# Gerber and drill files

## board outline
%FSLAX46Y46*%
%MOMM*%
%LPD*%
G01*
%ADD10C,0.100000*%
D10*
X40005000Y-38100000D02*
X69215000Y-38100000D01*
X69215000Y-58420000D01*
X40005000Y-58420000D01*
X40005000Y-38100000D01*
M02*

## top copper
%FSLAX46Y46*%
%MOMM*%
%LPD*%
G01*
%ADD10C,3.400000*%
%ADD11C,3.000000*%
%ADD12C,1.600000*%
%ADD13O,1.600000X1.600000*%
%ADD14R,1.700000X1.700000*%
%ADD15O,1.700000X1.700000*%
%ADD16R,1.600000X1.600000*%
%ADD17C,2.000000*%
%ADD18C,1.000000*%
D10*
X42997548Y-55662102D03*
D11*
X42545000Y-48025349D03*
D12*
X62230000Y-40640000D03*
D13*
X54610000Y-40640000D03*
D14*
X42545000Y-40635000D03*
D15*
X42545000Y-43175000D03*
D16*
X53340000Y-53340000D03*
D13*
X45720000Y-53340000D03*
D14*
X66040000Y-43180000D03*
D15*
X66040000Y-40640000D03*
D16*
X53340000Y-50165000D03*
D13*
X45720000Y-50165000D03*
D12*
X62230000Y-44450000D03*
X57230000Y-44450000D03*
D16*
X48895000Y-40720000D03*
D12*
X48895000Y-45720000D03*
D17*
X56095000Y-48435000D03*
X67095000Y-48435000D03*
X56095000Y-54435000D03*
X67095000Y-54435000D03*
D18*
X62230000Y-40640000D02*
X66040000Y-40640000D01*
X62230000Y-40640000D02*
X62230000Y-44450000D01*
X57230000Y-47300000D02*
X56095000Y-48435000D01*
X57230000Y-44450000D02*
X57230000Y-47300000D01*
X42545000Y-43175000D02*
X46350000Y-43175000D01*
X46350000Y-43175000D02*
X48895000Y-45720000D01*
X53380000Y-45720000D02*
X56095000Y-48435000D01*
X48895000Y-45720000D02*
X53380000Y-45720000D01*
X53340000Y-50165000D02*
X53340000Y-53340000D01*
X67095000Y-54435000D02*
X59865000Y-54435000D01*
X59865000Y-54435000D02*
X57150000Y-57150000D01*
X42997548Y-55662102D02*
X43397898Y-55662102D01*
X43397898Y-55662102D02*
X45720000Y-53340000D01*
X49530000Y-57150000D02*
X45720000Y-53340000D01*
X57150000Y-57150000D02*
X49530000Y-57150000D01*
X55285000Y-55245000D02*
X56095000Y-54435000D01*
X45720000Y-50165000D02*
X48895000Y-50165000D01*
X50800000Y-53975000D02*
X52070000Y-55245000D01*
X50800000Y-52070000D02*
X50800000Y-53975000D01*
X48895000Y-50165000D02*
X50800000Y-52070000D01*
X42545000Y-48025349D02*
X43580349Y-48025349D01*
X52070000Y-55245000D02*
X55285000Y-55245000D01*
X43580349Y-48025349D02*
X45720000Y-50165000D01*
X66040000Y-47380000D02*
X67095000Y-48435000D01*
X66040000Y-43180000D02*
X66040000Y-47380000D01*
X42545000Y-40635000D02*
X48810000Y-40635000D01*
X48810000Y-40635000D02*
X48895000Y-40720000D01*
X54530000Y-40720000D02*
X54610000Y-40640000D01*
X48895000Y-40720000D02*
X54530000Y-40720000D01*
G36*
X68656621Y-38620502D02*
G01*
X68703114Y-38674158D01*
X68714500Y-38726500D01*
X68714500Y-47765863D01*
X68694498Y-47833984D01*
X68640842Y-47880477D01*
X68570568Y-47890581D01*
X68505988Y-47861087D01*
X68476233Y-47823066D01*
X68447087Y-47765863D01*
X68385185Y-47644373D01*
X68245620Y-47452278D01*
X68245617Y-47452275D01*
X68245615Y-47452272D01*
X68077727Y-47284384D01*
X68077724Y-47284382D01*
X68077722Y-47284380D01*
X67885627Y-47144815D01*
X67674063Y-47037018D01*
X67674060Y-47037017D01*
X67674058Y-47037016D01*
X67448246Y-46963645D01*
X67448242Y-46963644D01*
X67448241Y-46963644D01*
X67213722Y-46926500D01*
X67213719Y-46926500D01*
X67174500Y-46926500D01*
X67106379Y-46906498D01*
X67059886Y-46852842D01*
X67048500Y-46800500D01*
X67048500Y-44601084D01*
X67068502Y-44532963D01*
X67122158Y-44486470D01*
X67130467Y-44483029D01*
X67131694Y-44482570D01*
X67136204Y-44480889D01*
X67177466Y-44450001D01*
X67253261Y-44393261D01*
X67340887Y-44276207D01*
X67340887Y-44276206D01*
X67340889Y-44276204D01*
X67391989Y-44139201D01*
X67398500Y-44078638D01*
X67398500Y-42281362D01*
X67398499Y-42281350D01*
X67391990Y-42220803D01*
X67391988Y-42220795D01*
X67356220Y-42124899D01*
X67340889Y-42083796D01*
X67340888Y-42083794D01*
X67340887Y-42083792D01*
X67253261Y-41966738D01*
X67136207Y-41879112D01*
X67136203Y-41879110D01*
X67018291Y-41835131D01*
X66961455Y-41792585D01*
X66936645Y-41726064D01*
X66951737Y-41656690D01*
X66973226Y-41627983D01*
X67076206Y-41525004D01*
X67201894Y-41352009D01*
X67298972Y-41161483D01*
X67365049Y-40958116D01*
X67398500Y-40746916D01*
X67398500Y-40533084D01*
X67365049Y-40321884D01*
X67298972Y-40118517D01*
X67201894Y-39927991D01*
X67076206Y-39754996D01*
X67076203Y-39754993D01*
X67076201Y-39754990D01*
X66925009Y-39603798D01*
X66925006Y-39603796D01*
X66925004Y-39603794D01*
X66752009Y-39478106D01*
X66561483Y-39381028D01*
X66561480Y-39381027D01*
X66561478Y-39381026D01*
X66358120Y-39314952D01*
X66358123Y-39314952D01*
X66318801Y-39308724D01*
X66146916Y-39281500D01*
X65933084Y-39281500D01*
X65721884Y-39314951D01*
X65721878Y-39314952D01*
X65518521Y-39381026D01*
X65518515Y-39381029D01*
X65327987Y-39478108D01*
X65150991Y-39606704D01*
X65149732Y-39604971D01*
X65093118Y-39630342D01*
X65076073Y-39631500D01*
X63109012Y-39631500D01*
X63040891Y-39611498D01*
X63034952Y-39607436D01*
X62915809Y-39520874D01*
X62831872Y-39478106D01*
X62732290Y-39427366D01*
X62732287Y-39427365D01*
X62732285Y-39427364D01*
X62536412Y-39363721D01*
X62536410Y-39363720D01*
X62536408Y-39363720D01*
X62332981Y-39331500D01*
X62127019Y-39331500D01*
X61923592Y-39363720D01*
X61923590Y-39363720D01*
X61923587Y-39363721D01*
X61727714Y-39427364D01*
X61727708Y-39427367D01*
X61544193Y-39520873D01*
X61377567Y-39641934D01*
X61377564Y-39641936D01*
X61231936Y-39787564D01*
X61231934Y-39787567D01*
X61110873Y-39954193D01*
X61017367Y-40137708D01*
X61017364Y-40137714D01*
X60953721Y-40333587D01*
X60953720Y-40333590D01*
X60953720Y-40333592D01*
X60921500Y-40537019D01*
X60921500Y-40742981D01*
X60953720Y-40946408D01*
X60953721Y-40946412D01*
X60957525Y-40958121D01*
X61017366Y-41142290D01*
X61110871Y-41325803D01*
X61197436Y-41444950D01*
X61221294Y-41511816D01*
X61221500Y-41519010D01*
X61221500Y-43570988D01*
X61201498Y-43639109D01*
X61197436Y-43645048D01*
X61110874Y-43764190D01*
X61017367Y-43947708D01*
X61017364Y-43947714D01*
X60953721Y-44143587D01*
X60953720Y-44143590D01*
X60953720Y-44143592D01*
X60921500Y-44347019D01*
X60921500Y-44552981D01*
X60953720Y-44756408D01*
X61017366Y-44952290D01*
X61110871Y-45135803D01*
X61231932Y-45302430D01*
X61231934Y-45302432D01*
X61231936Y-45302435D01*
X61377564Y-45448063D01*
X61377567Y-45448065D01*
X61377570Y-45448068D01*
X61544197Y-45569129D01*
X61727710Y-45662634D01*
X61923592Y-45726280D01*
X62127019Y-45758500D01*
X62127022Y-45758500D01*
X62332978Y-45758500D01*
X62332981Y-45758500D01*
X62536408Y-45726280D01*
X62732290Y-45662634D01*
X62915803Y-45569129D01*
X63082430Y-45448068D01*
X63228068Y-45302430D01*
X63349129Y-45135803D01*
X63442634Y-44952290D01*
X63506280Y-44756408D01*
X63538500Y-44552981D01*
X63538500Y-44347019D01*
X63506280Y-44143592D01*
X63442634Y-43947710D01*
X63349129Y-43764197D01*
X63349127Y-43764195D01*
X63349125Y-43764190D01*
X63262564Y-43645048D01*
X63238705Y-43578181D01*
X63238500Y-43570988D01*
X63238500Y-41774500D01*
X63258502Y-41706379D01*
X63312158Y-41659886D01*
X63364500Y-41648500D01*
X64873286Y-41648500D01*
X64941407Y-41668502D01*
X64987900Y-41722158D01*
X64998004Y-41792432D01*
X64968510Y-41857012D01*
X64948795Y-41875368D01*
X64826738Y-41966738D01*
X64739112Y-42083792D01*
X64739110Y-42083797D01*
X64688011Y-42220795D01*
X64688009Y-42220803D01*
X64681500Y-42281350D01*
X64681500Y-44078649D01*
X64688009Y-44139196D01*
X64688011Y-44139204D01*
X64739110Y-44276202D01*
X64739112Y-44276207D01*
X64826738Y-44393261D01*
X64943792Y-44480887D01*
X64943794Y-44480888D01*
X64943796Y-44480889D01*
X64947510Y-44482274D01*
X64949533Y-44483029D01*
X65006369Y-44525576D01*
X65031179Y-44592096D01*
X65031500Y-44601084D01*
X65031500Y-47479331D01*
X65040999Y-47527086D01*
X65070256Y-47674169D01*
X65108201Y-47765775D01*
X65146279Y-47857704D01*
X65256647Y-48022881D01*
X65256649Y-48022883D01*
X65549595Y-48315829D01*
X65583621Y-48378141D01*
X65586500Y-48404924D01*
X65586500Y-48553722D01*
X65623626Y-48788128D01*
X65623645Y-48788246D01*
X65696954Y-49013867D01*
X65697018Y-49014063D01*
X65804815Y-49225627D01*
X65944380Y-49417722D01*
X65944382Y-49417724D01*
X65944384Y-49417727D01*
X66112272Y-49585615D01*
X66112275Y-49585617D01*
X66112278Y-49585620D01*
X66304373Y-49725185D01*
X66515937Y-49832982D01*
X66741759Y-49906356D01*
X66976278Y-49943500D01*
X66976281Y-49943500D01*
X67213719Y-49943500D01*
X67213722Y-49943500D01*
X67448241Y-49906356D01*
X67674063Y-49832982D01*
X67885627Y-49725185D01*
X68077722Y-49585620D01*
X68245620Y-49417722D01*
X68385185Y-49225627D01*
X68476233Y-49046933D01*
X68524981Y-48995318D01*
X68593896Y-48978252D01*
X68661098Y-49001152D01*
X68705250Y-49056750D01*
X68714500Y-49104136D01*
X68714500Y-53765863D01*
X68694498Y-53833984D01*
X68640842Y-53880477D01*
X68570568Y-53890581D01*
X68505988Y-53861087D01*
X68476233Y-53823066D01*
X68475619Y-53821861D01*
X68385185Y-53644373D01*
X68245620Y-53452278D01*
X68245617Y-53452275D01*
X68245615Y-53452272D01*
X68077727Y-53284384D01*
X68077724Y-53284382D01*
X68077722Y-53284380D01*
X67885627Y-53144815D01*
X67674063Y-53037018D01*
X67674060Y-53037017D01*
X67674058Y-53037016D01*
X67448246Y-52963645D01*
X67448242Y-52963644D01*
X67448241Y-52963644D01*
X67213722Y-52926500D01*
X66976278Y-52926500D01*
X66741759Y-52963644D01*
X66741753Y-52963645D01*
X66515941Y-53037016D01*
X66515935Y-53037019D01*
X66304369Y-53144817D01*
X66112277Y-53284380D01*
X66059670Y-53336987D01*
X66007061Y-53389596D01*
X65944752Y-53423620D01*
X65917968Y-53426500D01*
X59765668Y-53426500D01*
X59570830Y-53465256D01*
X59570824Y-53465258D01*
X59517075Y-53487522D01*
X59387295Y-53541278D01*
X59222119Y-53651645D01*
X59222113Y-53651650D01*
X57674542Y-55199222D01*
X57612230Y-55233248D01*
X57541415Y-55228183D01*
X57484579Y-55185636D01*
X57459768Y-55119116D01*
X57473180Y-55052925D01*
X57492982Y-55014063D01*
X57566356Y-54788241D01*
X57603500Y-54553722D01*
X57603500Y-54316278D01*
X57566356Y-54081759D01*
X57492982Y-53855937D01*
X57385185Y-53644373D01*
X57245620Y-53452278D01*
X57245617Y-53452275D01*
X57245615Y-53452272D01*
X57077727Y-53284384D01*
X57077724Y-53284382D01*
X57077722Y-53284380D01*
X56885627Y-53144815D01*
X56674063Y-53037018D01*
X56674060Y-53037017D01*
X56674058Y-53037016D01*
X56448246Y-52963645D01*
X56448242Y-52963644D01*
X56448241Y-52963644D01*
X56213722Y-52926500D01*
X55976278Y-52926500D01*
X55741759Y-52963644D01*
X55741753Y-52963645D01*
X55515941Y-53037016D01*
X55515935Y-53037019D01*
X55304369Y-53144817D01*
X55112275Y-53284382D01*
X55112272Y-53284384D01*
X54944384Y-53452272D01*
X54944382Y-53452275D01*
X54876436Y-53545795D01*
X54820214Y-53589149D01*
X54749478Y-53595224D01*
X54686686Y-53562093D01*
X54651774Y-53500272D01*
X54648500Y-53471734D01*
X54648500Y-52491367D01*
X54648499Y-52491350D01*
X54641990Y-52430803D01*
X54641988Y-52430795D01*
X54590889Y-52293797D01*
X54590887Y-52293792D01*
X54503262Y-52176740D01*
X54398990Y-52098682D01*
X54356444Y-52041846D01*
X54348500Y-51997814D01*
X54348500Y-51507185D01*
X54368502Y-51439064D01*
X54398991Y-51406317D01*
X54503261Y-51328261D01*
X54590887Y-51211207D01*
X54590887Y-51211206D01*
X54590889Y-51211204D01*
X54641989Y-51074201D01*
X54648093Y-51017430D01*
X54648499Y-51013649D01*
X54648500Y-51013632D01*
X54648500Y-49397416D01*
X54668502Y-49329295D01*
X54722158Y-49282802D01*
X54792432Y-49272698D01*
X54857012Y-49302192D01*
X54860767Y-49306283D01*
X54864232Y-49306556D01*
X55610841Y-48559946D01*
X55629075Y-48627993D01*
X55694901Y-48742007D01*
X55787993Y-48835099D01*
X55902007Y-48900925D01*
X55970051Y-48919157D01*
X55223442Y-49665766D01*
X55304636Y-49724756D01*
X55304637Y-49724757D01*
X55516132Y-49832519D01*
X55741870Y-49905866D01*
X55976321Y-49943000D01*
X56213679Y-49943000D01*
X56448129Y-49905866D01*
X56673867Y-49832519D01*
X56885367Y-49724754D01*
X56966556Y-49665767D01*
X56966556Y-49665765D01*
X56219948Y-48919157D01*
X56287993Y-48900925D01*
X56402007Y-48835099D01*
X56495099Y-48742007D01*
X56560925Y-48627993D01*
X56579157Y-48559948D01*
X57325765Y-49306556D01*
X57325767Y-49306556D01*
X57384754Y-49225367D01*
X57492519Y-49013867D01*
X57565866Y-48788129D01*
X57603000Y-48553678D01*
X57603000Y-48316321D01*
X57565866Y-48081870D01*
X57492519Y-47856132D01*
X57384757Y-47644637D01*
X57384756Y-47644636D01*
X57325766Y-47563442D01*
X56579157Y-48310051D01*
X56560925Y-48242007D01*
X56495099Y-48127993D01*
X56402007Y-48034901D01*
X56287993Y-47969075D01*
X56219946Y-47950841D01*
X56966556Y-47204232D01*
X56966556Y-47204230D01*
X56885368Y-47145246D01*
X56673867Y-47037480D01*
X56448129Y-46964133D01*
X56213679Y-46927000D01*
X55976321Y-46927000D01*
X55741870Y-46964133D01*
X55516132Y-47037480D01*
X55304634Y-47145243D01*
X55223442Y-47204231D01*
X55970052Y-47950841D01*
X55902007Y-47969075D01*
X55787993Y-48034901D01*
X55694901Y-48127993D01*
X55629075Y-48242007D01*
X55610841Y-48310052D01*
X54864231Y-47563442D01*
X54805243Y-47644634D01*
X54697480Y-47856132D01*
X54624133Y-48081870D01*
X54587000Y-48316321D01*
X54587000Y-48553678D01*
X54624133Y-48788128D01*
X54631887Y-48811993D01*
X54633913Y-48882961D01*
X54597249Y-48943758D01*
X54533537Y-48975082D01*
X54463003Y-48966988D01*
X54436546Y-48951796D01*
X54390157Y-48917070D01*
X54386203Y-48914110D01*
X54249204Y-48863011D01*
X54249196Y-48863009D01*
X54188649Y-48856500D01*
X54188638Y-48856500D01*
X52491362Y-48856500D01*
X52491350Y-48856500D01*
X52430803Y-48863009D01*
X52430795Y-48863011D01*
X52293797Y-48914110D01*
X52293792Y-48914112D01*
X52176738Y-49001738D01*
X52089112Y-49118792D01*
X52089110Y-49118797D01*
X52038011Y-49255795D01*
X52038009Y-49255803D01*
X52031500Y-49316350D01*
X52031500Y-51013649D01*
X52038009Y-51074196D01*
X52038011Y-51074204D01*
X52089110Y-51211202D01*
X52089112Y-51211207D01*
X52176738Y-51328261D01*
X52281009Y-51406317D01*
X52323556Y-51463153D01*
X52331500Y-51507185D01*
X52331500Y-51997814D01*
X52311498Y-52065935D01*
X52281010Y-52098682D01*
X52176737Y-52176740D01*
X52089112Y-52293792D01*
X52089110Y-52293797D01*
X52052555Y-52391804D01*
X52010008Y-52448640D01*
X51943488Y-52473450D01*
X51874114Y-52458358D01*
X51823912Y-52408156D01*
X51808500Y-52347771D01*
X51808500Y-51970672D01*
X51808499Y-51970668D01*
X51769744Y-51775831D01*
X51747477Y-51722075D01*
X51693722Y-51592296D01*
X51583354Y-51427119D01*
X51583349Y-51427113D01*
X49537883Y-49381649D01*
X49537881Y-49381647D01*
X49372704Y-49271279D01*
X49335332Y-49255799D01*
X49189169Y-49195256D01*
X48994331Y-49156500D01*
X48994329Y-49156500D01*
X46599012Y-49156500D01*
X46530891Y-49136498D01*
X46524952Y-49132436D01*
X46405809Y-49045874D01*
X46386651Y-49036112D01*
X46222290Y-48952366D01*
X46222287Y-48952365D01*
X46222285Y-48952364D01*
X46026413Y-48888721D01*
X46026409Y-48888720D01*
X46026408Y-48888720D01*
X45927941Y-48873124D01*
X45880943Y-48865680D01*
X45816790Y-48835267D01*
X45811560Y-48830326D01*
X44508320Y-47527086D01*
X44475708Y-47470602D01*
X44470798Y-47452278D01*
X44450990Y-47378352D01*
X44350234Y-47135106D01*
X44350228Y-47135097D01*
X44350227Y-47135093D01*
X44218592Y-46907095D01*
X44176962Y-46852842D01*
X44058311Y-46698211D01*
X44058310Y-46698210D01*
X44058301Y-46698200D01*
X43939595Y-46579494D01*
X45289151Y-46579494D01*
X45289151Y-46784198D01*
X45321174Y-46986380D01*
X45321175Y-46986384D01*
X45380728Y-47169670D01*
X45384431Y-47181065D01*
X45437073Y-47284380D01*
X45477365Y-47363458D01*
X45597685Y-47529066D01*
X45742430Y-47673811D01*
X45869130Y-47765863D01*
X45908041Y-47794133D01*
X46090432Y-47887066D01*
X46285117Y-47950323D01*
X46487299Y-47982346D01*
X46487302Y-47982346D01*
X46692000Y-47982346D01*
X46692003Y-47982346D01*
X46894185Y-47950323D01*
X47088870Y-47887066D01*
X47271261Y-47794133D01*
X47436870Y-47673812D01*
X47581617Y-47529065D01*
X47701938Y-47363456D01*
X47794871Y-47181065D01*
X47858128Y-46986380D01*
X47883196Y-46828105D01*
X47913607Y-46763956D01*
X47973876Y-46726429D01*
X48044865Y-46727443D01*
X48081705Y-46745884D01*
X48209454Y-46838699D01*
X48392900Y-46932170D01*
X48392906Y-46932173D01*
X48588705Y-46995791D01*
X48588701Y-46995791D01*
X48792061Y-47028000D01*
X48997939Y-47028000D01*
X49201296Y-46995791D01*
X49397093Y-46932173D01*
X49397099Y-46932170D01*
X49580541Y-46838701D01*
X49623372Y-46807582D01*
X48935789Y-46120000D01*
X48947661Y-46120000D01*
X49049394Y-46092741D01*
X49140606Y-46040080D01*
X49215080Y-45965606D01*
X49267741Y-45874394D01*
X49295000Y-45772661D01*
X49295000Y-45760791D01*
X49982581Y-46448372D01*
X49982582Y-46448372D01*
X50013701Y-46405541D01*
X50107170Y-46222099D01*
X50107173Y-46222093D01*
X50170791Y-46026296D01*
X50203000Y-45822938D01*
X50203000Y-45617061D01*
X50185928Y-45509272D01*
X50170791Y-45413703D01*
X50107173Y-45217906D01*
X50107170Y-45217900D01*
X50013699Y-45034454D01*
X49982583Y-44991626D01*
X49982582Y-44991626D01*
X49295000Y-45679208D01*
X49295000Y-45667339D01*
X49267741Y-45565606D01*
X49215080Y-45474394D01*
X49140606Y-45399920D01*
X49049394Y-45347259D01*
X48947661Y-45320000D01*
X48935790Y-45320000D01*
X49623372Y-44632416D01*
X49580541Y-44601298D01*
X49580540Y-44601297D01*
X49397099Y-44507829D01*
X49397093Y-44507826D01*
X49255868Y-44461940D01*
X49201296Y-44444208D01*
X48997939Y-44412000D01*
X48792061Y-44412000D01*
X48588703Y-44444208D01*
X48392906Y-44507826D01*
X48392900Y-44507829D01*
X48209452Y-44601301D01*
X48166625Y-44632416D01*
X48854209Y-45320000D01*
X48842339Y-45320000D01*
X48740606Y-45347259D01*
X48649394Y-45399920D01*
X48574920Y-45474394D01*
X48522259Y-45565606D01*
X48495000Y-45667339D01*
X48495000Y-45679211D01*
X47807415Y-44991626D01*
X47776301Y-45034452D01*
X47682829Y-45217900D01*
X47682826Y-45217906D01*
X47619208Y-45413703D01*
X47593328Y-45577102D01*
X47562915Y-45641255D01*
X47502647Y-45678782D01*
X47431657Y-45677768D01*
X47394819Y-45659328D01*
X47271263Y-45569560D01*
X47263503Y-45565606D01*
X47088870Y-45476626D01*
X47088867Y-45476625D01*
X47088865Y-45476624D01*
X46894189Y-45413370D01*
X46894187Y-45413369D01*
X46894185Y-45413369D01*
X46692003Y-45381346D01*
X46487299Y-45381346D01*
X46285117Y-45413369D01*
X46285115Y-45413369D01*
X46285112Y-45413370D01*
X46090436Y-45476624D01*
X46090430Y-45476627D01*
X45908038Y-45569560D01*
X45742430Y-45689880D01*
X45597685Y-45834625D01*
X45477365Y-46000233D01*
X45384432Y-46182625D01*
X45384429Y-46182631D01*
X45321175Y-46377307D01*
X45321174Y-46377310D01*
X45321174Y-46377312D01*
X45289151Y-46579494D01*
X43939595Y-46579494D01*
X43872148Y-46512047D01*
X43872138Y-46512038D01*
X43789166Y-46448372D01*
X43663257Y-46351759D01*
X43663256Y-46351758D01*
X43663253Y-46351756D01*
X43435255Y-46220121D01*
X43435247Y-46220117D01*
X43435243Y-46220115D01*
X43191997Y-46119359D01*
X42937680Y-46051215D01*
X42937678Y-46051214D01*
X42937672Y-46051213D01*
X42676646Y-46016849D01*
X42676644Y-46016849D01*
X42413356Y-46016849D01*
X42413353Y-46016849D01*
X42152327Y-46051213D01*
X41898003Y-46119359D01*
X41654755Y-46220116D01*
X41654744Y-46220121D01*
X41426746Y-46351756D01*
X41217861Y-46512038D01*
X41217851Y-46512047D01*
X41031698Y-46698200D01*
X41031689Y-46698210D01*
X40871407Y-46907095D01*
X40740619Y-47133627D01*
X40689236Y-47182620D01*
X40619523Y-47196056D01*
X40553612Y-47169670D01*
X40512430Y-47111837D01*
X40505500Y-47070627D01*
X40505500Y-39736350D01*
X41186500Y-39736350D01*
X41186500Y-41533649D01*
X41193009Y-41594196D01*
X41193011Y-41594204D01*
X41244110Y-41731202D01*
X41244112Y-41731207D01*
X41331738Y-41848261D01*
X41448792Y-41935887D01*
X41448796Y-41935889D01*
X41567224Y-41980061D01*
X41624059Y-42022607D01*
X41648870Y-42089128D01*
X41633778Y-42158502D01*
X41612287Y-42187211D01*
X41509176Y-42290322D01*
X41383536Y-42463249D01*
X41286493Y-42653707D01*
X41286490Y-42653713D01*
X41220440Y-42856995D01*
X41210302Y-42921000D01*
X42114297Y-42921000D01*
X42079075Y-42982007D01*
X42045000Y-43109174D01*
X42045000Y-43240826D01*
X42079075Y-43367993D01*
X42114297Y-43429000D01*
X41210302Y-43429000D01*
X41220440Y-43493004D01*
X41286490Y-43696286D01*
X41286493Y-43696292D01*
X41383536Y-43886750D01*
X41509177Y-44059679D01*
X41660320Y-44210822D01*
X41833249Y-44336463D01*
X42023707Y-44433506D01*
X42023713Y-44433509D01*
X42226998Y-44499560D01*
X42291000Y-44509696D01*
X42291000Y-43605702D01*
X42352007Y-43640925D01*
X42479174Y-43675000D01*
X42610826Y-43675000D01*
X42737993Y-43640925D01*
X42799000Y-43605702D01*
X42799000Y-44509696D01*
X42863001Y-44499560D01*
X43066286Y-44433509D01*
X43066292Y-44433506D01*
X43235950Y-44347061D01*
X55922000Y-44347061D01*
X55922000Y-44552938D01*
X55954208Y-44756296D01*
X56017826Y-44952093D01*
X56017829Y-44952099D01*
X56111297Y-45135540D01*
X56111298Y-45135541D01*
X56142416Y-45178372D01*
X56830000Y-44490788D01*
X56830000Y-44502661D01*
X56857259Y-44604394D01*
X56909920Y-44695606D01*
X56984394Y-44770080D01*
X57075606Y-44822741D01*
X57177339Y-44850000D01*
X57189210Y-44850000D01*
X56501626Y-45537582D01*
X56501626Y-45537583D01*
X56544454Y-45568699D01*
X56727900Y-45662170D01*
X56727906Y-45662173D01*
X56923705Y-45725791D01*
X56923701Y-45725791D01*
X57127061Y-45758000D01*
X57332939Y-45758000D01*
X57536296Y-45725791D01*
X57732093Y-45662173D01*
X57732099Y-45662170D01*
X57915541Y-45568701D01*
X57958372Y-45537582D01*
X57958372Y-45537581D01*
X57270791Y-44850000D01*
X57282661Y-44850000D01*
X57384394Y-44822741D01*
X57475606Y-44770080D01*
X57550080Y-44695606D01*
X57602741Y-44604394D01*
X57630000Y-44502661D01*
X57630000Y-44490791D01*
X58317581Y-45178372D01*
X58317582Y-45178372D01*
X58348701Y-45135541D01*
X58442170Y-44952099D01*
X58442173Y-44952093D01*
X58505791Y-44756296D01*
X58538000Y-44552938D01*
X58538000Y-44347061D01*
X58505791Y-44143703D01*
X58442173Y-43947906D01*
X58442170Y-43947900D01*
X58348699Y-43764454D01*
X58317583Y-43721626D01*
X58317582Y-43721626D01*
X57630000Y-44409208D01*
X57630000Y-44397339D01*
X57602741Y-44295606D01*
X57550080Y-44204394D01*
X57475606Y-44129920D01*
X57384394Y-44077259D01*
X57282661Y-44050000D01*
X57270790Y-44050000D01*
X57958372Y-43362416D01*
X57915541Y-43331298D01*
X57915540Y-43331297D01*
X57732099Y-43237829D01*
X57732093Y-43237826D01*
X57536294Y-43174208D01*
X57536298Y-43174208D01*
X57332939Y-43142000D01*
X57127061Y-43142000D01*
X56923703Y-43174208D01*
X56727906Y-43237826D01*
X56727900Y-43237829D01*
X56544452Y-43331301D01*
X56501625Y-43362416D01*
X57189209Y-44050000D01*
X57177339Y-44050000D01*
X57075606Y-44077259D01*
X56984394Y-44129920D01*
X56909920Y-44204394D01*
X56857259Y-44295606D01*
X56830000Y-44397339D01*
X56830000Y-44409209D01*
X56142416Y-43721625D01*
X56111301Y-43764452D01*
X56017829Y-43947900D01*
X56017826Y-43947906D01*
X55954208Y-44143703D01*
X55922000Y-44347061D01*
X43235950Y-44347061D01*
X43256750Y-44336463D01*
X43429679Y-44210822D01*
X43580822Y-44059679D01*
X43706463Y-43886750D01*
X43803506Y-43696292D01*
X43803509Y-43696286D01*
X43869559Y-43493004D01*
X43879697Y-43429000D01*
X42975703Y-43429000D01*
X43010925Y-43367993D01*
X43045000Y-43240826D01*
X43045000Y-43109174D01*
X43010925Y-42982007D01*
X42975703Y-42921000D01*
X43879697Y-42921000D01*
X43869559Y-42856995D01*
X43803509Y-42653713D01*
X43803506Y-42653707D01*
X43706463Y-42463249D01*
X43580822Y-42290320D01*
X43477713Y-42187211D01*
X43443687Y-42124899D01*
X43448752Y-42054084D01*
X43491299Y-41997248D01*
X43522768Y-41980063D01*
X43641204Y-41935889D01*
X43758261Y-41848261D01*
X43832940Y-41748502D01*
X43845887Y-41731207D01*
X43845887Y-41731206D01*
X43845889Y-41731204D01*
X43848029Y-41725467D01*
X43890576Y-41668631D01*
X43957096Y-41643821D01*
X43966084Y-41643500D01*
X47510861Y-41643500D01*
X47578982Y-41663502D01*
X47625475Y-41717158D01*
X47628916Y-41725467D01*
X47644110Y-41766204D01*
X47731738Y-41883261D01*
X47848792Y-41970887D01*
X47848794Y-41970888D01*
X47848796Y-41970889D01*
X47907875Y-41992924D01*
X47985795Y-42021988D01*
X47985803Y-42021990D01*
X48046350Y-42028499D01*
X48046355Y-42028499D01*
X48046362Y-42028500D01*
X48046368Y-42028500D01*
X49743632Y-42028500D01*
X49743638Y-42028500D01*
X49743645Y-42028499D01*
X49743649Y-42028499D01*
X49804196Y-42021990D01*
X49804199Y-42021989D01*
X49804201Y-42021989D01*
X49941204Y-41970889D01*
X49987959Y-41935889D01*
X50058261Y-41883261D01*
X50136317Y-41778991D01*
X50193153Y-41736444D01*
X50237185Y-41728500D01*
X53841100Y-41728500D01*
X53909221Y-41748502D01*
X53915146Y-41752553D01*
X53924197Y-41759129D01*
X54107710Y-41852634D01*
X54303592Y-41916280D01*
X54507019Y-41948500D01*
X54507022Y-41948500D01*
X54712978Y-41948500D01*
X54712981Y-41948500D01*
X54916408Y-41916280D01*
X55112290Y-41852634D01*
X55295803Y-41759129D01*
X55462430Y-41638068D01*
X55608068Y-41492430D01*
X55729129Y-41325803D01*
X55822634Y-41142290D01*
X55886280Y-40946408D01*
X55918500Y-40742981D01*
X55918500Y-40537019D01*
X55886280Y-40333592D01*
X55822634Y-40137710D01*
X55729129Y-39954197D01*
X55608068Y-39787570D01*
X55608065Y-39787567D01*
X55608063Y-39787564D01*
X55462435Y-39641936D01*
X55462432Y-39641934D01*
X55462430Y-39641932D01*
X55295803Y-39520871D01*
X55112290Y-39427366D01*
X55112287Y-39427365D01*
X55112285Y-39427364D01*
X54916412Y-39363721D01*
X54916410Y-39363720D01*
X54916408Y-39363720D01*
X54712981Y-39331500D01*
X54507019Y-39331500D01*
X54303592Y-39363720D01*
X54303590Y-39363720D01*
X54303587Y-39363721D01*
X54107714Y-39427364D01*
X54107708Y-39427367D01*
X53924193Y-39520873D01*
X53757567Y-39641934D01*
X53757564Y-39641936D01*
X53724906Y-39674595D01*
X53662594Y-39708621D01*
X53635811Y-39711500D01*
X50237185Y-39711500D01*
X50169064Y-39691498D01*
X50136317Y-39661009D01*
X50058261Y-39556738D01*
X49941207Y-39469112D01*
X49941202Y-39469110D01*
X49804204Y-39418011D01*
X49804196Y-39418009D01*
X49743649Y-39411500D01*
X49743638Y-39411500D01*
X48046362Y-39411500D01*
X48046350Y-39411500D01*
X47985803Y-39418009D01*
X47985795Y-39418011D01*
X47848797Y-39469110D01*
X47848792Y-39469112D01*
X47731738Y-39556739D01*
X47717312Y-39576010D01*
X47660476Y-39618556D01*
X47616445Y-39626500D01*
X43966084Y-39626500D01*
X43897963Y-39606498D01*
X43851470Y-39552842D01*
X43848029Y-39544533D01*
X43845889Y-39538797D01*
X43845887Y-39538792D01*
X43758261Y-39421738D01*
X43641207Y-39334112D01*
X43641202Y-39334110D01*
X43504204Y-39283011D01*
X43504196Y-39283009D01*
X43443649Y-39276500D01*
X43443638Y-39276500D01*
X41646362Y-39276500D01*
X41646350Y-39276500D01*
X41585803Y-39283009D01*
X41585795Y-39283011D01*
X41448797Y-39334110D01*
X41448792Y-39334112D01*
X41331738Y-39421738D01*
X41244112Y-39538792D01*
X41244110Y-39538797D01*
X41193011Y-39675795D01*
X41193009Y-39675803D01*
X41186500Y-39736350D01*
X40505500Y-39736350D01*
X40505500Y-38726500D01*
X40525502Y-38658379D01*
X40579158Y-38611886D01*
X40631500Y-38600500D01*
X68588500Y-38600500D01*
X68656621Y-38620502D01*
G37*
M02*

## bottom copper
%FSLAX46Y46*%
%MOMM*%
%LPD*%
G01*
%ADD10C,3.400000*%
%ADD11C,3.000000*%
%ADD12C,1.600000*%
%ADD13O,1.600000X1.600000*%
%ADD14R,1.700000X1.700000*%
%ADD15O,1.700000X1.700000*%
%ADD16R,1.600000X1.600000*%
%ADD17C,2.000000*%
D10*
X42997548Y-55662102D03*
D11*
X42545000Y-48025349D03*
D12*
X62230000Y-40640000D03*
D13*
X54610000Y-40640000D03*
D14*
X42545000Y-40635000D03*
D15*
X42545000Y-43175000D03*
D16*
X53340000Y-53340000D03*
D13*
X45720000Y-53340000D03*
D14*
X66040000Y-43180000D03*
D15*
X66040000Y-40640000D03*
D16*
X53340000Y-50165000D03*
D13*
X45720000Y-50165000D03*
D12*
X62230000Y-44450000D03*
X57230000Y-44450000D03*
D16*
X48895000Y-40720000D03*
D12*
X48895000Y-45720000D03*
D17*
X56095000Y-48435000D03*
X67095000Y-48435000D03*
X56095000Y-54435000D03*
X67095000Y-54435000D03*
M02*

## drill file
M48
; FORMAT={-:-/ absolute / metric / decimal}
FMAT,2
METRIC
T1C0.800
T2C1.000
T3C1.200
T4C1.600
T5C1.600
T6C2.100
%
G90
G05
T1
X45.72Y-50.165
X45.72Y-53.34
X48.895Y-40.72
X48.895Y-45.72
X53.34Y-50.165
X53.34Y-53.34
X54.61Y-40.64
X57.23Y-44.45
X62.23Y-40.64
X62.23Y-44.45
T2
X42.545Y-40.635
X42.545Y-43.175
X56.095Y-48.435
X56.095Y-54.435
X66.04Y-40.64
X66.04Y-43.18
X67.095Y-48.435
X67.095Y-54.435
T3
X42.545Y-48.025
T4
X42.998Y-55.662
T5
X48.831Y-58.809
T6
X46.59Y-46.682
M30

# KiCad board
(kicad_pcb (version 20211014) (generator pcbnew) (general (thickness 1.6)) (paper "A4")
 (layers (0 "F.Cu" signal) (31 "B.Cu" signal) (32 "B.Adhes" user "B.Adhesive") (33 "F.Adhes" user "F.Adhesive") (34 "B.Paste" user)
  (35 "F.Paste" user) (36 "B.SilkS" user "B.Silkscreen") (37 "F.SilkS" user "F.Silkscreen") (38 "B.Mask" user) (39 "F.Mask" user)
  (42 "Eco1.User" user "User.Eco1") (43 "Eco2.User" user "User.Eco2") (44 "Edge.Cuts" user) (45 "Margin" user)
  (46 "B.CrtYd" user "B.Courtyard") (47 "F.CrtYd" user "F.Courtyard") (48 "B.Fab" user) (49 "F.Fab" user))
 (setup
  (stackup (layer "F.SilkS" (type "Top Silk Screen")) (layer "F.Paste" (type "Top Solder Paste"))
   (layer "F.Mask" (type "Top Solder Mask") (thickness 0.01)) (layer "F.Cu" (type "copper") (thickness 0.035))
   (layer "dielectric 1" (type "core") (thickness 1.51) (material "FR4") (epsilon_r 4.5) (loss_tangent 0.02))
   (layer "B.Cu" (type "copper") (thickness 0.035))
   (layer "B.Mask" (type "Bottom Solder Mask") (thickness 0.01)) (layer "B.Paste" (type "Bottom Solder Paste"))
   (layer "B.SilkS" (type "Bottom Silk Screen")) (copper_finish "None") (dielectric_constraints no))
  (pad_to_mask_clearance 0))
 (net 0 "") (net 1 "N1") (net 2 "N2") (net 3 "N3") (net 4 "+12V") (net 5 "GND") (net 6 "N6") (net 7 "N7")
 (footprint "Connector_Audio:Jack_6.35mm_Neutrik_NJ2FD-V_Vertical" (layer "F.Cu") (at 42.545 48.025349 45)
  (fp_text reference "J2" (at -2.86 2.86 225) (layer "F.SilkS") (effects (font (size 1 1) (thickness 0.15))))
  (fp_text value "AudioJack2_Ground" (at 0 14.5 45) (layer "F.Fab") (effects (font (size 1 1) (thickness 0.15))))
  (pad "" np_thru_hole circle (at -3.18 12.07 225) (size 1.6 1.6) (drill 1.6) (layers *.Cu *.Mask))
  (pad "" np_thru_hole circle (at 3.81 1.91 225) (size 2.1 2.1) (drill 2.1) (layers *.Cu *.Mask))
  (pad "S" thru_hole circle (at -5.08 5.72 225) (size 3.4 3.4) (drill 1.6) (layers *.Cu *.Mask) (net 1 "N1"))
  (pad "T" thru_hole circle (at 0 0 225) (size 3 3) (drill 1.2) (layers *.Cu *.Mask) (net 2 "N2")))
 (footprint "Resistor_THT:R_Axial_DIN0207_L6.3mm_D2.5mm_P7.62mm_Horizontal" (layer "F.Cu") (at 62.23 40.64 180)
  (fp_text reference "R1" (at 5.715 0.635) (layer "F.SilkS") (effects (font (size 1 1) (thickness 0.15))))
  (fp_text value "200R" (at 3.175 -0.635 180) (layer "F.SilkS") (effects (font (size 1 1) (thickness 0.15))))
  (pad "1" thru_hole circle (at 0 0 180) (size 1.6 1.6) (drill 0.8) (layers *.Cu *.Mask) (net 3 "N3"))
  (pad "2" thru_hole oval (at 7.62 0 180) (size 1.6 1.6) (drill 0.8) (layers *.Cu *.Mask) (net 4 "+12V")))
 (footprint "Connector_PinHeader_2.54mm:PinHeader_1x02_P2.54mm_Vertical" (layer "F.Cu") (at 42.545 40.635)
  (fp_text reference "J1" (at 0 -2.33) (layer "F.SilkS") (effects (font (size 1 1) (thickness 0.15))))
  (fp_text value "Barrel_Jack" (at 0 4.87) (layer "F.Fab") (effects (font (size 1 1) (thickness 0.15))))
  (pad "1" thru_hole rect (at 0 0) (size 1.7 1.7) (drill 1) (layers *.Cu *.Mask) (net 4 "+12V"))
  (pad "2" thru_hole oval (at 0 2.54) (size 1.7 1.7) (drill 1) (layers *.Cu *.Mask) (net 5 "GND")))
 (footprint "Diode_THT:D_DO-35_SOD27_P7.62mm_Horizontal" (layer "F.Cu") (at 53.34 53.34 180)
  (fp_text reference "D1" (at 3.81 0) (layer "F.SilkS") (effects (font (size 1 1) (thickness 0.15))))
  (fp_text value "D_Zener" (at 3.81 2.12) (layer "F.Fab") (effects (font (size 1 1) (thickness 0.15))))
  (pad "1" thru_hole rect (at 0 0 180) (size 1.6 1.6) (drill 0.8) (layers *.Cu *.Mask) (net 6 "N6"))
  (pad "2" thru_hole oval (at 7.62 0 180) (size 1.6 1.6) (drill 0.8) (layers *.Cu *.Mask) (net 1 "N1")))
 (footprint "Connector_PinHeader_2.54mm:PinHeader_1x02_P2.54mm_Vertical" (layer "F.Cu") (at 66.04 43.18 180)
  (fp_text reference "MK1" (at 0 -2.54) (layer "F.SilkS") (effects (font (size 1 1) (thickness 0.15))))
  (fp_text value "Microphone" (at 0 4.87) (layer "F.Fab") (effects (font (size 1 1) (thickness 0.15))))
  (pad "1" thru_hole rect (at 0 0 180) (size 1.7 1.7) (drill 1) (layers *.Cu *.Mask) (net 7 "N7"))
  (pad "2" thru_hole oval (at 0 2.54 180) (size 1.7 1.7) (drill 1) (layers *.Cu *.Mask) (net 3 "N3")))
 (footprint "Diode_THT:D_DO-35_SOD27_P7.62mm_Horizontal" (layer "F.Cu") (at 53.34 50.165 180)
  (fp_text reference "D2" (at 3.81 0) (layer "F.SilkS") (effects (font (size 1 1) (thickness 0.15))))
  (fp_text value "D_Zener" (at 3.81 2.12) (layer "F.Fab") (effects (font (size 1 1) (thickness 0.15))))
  (pad "1" thru_hole rect (at 0 0 180) (size 1.6 1.6) (drill 0.8) (layers *.Cu *.Mask) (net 6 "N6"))
  (pad "2" thru_hole oval (at 7.62 0 180) (size 1.6 1.6) (drill 0.8) (layers *.Cu *.Mask) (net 2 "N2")))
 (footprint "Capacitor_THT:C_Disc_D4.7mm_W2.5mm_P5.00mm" (layer "F.Cu") (at 62.23 44.45 180)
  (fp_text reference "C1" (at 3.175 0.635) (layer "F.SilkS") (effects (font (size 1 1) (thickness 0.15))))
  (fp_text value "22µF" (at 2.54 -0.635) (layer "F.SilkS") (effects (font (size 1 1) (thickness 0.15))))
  (pad "1" thru_hole circle (at 0 0 180) (size 1.6 1.6) (drill 0.8) (layers *.Cu *.Mask) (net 3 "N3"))
  (pad "2" thru_hole circle (at 5 0 180) (size 1.6 1.6) (drill 0.8) (layers *.Cu *.Mask) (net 5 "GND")))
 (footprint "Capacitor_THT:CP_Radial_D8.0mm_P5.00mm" (layer "F.Cu") (at 48.895 40.72 -90)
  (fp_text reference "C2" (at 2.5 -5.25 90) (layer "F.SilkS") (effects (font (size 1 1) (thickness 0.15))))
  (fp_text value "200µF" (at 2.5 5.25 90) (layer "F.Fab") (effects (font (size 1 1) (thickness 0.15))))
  (pad "1" thru_hole rect (at 0 0 270) (size 1.6 1.6) (drill 0.8) (layers *.Cu *.Mask) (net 4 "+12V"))
  (pad "2" thru_hole circle (at 5 0 270) (size 1.6 1.6) (drill 0.8) (layers *.Cu *.Mask) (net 5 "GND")))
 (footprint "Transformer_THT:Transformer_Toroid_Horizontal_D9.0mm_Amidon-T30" (layer "B.Cu") (at 56.095 48.435)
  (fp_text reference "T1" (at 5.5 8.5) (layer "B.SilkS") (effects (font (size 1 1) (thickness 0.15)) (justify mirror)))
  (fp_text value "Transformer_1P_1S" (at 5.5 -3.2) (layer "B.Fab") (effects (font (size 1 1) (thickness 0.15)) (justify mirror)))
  (pad "1" thru_hole circle (at 0 0) (size 2 2) (drill 1) (layers *.Cu *.Mask) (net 5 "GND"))
  (pad "2" thru_hole circle (at 11 0) (size 2 2) (drill 1) (layers *.Cu *.Mask) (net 7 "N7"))
  (pad "3" thru_hole circle (at 0 6) (size 2 2) (drill 1) (layers *.Cu *.Mask) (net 2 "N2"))
  (pad "4" thru_hole circle (at 11 6) (size 2 2) (drill 1) (layers *.Cu *.Mask) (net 1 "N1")))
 (gr_rect (start 40.005 38.1) (end 69.215 58.42) (layer "Edge.Cuts") (width 0.1) (fill none))
 (segment (start 62.23 40.64) (end 66.04 40.64) (width 1) (layer "F.Cu") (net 3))
 (segment (start 62.23 40.64) (end 62.23 44.45) (width 1) (layer "F.Cu") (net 3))
 (segment (start 57.23 47.3) (end 56.095 48.435) (width 1) (layer "F.Cu") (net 5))
 (segment (start 57.23 44.45) (end 57.23 47.3) (width 1) (layer "F.Cu") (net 5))
 (segment (start 42.545 43.175) (end 46.35 43.175) (width 1) (layer "F.Cu") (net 5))
 (segment (start 46.35 43.175) (end 48.895 45.72) (width 1) (layer "F.Cu") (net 5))
 (segment (start 53.38 45.72) (end 56.095 48.435) (width 1) (layer "F.Cu") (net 5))
 (segment (start 48.895 45.72) (end 53.38 45.72) (width 1) (layer "F.Cu") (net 5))
 (segment (start 53.34 50.165) (end 53.34 53.34) (width 1) (layer "F.Cu") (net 6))
 (segment (start 67.095 54.435) (end 59.865 54.435) (width 1) (layer "F.Cu") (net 1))
 (segment (start 59.865 54.435) (end 57.15 57.15) (width 1) (layer "F.Cu") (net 1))
 (segment (start 42.997548 55.662102) (end 43.397898 55.662102) (width 1) (layer "F.Cu") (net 1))
 (segment (start 43.397898 55.662102) (end 45.72 53.34) (width 1) (layer "F.Cu") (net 1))
 (segment (start 49.53 57.15) (end 45.72 53.34) (width 1) (layer "F.Cu") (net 1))
 (segment (start 57.15 57.15) (end 49.53 57.15) (width 1) (layer "F.Cu") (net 1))
 (segment (start 55.285 55.245) (end 56.095 54.435) (width 1) (layer "F.Cu") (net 2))
 (segment (start 45.72 50.165) (end 48.895 50.165) (width 1) (layer "F.Cu") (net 2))
 (segment (start 50.8 53.975) (end 52.07 55.245) (width 1) (layer "F.Cu") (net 2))
 (segment (start 50.8 52.07) (end 50.8 53.975) (width 1) (layer "F.Cu") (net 2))
 (segment (start 48.895 50.165) (end 50.8 52.07) (width 1) (layer "F.Cu") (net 2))
 (segment (start 42.545 48.025349) (end 43.580349 48.025349) (width 1) (layer "F.Cu") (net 2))
 (segment (start 52.07 55.245) (end 55.285 55.245) (width 1) (layer "F.Cu") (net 2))
 (segment (start 43.580349 48.025349) (end 45.72 50.165) (width 1) (layer "F.Cu") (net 2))
 (segment (start 66.04 47.38) (end 67.095 48.435) (width 1) (layer "F.Cu") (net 7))
 (segment (start 66.04 43.18) (end 66.04 47.38) (width 1) (layer "F.Cu") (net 7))
 (segment (start 42.545 40.635) (end 48.81 40.635) (width 1) (layer "F.Cu") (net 4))
 (segment (start 48.81 40.635) (end 48.895 40.72) (width 1) (layer "F.Cu") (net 4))
 (segment (start 54.53 40.72) (end 54.61 40.64) (width 1) (layer "F.Cu") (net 4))
 (segment (start 48.895 40.72) (end 54.53 40.72) (width 1) (layer "F.Cu") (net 4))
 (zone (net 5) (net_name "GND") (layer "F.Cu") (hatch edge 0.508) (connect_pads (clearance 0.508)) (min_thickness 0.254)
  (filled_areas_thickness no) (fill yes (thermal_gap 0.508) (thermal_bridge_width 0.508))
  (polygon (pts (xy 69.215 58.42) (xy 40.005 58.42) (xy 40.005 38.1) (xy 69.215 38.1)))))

